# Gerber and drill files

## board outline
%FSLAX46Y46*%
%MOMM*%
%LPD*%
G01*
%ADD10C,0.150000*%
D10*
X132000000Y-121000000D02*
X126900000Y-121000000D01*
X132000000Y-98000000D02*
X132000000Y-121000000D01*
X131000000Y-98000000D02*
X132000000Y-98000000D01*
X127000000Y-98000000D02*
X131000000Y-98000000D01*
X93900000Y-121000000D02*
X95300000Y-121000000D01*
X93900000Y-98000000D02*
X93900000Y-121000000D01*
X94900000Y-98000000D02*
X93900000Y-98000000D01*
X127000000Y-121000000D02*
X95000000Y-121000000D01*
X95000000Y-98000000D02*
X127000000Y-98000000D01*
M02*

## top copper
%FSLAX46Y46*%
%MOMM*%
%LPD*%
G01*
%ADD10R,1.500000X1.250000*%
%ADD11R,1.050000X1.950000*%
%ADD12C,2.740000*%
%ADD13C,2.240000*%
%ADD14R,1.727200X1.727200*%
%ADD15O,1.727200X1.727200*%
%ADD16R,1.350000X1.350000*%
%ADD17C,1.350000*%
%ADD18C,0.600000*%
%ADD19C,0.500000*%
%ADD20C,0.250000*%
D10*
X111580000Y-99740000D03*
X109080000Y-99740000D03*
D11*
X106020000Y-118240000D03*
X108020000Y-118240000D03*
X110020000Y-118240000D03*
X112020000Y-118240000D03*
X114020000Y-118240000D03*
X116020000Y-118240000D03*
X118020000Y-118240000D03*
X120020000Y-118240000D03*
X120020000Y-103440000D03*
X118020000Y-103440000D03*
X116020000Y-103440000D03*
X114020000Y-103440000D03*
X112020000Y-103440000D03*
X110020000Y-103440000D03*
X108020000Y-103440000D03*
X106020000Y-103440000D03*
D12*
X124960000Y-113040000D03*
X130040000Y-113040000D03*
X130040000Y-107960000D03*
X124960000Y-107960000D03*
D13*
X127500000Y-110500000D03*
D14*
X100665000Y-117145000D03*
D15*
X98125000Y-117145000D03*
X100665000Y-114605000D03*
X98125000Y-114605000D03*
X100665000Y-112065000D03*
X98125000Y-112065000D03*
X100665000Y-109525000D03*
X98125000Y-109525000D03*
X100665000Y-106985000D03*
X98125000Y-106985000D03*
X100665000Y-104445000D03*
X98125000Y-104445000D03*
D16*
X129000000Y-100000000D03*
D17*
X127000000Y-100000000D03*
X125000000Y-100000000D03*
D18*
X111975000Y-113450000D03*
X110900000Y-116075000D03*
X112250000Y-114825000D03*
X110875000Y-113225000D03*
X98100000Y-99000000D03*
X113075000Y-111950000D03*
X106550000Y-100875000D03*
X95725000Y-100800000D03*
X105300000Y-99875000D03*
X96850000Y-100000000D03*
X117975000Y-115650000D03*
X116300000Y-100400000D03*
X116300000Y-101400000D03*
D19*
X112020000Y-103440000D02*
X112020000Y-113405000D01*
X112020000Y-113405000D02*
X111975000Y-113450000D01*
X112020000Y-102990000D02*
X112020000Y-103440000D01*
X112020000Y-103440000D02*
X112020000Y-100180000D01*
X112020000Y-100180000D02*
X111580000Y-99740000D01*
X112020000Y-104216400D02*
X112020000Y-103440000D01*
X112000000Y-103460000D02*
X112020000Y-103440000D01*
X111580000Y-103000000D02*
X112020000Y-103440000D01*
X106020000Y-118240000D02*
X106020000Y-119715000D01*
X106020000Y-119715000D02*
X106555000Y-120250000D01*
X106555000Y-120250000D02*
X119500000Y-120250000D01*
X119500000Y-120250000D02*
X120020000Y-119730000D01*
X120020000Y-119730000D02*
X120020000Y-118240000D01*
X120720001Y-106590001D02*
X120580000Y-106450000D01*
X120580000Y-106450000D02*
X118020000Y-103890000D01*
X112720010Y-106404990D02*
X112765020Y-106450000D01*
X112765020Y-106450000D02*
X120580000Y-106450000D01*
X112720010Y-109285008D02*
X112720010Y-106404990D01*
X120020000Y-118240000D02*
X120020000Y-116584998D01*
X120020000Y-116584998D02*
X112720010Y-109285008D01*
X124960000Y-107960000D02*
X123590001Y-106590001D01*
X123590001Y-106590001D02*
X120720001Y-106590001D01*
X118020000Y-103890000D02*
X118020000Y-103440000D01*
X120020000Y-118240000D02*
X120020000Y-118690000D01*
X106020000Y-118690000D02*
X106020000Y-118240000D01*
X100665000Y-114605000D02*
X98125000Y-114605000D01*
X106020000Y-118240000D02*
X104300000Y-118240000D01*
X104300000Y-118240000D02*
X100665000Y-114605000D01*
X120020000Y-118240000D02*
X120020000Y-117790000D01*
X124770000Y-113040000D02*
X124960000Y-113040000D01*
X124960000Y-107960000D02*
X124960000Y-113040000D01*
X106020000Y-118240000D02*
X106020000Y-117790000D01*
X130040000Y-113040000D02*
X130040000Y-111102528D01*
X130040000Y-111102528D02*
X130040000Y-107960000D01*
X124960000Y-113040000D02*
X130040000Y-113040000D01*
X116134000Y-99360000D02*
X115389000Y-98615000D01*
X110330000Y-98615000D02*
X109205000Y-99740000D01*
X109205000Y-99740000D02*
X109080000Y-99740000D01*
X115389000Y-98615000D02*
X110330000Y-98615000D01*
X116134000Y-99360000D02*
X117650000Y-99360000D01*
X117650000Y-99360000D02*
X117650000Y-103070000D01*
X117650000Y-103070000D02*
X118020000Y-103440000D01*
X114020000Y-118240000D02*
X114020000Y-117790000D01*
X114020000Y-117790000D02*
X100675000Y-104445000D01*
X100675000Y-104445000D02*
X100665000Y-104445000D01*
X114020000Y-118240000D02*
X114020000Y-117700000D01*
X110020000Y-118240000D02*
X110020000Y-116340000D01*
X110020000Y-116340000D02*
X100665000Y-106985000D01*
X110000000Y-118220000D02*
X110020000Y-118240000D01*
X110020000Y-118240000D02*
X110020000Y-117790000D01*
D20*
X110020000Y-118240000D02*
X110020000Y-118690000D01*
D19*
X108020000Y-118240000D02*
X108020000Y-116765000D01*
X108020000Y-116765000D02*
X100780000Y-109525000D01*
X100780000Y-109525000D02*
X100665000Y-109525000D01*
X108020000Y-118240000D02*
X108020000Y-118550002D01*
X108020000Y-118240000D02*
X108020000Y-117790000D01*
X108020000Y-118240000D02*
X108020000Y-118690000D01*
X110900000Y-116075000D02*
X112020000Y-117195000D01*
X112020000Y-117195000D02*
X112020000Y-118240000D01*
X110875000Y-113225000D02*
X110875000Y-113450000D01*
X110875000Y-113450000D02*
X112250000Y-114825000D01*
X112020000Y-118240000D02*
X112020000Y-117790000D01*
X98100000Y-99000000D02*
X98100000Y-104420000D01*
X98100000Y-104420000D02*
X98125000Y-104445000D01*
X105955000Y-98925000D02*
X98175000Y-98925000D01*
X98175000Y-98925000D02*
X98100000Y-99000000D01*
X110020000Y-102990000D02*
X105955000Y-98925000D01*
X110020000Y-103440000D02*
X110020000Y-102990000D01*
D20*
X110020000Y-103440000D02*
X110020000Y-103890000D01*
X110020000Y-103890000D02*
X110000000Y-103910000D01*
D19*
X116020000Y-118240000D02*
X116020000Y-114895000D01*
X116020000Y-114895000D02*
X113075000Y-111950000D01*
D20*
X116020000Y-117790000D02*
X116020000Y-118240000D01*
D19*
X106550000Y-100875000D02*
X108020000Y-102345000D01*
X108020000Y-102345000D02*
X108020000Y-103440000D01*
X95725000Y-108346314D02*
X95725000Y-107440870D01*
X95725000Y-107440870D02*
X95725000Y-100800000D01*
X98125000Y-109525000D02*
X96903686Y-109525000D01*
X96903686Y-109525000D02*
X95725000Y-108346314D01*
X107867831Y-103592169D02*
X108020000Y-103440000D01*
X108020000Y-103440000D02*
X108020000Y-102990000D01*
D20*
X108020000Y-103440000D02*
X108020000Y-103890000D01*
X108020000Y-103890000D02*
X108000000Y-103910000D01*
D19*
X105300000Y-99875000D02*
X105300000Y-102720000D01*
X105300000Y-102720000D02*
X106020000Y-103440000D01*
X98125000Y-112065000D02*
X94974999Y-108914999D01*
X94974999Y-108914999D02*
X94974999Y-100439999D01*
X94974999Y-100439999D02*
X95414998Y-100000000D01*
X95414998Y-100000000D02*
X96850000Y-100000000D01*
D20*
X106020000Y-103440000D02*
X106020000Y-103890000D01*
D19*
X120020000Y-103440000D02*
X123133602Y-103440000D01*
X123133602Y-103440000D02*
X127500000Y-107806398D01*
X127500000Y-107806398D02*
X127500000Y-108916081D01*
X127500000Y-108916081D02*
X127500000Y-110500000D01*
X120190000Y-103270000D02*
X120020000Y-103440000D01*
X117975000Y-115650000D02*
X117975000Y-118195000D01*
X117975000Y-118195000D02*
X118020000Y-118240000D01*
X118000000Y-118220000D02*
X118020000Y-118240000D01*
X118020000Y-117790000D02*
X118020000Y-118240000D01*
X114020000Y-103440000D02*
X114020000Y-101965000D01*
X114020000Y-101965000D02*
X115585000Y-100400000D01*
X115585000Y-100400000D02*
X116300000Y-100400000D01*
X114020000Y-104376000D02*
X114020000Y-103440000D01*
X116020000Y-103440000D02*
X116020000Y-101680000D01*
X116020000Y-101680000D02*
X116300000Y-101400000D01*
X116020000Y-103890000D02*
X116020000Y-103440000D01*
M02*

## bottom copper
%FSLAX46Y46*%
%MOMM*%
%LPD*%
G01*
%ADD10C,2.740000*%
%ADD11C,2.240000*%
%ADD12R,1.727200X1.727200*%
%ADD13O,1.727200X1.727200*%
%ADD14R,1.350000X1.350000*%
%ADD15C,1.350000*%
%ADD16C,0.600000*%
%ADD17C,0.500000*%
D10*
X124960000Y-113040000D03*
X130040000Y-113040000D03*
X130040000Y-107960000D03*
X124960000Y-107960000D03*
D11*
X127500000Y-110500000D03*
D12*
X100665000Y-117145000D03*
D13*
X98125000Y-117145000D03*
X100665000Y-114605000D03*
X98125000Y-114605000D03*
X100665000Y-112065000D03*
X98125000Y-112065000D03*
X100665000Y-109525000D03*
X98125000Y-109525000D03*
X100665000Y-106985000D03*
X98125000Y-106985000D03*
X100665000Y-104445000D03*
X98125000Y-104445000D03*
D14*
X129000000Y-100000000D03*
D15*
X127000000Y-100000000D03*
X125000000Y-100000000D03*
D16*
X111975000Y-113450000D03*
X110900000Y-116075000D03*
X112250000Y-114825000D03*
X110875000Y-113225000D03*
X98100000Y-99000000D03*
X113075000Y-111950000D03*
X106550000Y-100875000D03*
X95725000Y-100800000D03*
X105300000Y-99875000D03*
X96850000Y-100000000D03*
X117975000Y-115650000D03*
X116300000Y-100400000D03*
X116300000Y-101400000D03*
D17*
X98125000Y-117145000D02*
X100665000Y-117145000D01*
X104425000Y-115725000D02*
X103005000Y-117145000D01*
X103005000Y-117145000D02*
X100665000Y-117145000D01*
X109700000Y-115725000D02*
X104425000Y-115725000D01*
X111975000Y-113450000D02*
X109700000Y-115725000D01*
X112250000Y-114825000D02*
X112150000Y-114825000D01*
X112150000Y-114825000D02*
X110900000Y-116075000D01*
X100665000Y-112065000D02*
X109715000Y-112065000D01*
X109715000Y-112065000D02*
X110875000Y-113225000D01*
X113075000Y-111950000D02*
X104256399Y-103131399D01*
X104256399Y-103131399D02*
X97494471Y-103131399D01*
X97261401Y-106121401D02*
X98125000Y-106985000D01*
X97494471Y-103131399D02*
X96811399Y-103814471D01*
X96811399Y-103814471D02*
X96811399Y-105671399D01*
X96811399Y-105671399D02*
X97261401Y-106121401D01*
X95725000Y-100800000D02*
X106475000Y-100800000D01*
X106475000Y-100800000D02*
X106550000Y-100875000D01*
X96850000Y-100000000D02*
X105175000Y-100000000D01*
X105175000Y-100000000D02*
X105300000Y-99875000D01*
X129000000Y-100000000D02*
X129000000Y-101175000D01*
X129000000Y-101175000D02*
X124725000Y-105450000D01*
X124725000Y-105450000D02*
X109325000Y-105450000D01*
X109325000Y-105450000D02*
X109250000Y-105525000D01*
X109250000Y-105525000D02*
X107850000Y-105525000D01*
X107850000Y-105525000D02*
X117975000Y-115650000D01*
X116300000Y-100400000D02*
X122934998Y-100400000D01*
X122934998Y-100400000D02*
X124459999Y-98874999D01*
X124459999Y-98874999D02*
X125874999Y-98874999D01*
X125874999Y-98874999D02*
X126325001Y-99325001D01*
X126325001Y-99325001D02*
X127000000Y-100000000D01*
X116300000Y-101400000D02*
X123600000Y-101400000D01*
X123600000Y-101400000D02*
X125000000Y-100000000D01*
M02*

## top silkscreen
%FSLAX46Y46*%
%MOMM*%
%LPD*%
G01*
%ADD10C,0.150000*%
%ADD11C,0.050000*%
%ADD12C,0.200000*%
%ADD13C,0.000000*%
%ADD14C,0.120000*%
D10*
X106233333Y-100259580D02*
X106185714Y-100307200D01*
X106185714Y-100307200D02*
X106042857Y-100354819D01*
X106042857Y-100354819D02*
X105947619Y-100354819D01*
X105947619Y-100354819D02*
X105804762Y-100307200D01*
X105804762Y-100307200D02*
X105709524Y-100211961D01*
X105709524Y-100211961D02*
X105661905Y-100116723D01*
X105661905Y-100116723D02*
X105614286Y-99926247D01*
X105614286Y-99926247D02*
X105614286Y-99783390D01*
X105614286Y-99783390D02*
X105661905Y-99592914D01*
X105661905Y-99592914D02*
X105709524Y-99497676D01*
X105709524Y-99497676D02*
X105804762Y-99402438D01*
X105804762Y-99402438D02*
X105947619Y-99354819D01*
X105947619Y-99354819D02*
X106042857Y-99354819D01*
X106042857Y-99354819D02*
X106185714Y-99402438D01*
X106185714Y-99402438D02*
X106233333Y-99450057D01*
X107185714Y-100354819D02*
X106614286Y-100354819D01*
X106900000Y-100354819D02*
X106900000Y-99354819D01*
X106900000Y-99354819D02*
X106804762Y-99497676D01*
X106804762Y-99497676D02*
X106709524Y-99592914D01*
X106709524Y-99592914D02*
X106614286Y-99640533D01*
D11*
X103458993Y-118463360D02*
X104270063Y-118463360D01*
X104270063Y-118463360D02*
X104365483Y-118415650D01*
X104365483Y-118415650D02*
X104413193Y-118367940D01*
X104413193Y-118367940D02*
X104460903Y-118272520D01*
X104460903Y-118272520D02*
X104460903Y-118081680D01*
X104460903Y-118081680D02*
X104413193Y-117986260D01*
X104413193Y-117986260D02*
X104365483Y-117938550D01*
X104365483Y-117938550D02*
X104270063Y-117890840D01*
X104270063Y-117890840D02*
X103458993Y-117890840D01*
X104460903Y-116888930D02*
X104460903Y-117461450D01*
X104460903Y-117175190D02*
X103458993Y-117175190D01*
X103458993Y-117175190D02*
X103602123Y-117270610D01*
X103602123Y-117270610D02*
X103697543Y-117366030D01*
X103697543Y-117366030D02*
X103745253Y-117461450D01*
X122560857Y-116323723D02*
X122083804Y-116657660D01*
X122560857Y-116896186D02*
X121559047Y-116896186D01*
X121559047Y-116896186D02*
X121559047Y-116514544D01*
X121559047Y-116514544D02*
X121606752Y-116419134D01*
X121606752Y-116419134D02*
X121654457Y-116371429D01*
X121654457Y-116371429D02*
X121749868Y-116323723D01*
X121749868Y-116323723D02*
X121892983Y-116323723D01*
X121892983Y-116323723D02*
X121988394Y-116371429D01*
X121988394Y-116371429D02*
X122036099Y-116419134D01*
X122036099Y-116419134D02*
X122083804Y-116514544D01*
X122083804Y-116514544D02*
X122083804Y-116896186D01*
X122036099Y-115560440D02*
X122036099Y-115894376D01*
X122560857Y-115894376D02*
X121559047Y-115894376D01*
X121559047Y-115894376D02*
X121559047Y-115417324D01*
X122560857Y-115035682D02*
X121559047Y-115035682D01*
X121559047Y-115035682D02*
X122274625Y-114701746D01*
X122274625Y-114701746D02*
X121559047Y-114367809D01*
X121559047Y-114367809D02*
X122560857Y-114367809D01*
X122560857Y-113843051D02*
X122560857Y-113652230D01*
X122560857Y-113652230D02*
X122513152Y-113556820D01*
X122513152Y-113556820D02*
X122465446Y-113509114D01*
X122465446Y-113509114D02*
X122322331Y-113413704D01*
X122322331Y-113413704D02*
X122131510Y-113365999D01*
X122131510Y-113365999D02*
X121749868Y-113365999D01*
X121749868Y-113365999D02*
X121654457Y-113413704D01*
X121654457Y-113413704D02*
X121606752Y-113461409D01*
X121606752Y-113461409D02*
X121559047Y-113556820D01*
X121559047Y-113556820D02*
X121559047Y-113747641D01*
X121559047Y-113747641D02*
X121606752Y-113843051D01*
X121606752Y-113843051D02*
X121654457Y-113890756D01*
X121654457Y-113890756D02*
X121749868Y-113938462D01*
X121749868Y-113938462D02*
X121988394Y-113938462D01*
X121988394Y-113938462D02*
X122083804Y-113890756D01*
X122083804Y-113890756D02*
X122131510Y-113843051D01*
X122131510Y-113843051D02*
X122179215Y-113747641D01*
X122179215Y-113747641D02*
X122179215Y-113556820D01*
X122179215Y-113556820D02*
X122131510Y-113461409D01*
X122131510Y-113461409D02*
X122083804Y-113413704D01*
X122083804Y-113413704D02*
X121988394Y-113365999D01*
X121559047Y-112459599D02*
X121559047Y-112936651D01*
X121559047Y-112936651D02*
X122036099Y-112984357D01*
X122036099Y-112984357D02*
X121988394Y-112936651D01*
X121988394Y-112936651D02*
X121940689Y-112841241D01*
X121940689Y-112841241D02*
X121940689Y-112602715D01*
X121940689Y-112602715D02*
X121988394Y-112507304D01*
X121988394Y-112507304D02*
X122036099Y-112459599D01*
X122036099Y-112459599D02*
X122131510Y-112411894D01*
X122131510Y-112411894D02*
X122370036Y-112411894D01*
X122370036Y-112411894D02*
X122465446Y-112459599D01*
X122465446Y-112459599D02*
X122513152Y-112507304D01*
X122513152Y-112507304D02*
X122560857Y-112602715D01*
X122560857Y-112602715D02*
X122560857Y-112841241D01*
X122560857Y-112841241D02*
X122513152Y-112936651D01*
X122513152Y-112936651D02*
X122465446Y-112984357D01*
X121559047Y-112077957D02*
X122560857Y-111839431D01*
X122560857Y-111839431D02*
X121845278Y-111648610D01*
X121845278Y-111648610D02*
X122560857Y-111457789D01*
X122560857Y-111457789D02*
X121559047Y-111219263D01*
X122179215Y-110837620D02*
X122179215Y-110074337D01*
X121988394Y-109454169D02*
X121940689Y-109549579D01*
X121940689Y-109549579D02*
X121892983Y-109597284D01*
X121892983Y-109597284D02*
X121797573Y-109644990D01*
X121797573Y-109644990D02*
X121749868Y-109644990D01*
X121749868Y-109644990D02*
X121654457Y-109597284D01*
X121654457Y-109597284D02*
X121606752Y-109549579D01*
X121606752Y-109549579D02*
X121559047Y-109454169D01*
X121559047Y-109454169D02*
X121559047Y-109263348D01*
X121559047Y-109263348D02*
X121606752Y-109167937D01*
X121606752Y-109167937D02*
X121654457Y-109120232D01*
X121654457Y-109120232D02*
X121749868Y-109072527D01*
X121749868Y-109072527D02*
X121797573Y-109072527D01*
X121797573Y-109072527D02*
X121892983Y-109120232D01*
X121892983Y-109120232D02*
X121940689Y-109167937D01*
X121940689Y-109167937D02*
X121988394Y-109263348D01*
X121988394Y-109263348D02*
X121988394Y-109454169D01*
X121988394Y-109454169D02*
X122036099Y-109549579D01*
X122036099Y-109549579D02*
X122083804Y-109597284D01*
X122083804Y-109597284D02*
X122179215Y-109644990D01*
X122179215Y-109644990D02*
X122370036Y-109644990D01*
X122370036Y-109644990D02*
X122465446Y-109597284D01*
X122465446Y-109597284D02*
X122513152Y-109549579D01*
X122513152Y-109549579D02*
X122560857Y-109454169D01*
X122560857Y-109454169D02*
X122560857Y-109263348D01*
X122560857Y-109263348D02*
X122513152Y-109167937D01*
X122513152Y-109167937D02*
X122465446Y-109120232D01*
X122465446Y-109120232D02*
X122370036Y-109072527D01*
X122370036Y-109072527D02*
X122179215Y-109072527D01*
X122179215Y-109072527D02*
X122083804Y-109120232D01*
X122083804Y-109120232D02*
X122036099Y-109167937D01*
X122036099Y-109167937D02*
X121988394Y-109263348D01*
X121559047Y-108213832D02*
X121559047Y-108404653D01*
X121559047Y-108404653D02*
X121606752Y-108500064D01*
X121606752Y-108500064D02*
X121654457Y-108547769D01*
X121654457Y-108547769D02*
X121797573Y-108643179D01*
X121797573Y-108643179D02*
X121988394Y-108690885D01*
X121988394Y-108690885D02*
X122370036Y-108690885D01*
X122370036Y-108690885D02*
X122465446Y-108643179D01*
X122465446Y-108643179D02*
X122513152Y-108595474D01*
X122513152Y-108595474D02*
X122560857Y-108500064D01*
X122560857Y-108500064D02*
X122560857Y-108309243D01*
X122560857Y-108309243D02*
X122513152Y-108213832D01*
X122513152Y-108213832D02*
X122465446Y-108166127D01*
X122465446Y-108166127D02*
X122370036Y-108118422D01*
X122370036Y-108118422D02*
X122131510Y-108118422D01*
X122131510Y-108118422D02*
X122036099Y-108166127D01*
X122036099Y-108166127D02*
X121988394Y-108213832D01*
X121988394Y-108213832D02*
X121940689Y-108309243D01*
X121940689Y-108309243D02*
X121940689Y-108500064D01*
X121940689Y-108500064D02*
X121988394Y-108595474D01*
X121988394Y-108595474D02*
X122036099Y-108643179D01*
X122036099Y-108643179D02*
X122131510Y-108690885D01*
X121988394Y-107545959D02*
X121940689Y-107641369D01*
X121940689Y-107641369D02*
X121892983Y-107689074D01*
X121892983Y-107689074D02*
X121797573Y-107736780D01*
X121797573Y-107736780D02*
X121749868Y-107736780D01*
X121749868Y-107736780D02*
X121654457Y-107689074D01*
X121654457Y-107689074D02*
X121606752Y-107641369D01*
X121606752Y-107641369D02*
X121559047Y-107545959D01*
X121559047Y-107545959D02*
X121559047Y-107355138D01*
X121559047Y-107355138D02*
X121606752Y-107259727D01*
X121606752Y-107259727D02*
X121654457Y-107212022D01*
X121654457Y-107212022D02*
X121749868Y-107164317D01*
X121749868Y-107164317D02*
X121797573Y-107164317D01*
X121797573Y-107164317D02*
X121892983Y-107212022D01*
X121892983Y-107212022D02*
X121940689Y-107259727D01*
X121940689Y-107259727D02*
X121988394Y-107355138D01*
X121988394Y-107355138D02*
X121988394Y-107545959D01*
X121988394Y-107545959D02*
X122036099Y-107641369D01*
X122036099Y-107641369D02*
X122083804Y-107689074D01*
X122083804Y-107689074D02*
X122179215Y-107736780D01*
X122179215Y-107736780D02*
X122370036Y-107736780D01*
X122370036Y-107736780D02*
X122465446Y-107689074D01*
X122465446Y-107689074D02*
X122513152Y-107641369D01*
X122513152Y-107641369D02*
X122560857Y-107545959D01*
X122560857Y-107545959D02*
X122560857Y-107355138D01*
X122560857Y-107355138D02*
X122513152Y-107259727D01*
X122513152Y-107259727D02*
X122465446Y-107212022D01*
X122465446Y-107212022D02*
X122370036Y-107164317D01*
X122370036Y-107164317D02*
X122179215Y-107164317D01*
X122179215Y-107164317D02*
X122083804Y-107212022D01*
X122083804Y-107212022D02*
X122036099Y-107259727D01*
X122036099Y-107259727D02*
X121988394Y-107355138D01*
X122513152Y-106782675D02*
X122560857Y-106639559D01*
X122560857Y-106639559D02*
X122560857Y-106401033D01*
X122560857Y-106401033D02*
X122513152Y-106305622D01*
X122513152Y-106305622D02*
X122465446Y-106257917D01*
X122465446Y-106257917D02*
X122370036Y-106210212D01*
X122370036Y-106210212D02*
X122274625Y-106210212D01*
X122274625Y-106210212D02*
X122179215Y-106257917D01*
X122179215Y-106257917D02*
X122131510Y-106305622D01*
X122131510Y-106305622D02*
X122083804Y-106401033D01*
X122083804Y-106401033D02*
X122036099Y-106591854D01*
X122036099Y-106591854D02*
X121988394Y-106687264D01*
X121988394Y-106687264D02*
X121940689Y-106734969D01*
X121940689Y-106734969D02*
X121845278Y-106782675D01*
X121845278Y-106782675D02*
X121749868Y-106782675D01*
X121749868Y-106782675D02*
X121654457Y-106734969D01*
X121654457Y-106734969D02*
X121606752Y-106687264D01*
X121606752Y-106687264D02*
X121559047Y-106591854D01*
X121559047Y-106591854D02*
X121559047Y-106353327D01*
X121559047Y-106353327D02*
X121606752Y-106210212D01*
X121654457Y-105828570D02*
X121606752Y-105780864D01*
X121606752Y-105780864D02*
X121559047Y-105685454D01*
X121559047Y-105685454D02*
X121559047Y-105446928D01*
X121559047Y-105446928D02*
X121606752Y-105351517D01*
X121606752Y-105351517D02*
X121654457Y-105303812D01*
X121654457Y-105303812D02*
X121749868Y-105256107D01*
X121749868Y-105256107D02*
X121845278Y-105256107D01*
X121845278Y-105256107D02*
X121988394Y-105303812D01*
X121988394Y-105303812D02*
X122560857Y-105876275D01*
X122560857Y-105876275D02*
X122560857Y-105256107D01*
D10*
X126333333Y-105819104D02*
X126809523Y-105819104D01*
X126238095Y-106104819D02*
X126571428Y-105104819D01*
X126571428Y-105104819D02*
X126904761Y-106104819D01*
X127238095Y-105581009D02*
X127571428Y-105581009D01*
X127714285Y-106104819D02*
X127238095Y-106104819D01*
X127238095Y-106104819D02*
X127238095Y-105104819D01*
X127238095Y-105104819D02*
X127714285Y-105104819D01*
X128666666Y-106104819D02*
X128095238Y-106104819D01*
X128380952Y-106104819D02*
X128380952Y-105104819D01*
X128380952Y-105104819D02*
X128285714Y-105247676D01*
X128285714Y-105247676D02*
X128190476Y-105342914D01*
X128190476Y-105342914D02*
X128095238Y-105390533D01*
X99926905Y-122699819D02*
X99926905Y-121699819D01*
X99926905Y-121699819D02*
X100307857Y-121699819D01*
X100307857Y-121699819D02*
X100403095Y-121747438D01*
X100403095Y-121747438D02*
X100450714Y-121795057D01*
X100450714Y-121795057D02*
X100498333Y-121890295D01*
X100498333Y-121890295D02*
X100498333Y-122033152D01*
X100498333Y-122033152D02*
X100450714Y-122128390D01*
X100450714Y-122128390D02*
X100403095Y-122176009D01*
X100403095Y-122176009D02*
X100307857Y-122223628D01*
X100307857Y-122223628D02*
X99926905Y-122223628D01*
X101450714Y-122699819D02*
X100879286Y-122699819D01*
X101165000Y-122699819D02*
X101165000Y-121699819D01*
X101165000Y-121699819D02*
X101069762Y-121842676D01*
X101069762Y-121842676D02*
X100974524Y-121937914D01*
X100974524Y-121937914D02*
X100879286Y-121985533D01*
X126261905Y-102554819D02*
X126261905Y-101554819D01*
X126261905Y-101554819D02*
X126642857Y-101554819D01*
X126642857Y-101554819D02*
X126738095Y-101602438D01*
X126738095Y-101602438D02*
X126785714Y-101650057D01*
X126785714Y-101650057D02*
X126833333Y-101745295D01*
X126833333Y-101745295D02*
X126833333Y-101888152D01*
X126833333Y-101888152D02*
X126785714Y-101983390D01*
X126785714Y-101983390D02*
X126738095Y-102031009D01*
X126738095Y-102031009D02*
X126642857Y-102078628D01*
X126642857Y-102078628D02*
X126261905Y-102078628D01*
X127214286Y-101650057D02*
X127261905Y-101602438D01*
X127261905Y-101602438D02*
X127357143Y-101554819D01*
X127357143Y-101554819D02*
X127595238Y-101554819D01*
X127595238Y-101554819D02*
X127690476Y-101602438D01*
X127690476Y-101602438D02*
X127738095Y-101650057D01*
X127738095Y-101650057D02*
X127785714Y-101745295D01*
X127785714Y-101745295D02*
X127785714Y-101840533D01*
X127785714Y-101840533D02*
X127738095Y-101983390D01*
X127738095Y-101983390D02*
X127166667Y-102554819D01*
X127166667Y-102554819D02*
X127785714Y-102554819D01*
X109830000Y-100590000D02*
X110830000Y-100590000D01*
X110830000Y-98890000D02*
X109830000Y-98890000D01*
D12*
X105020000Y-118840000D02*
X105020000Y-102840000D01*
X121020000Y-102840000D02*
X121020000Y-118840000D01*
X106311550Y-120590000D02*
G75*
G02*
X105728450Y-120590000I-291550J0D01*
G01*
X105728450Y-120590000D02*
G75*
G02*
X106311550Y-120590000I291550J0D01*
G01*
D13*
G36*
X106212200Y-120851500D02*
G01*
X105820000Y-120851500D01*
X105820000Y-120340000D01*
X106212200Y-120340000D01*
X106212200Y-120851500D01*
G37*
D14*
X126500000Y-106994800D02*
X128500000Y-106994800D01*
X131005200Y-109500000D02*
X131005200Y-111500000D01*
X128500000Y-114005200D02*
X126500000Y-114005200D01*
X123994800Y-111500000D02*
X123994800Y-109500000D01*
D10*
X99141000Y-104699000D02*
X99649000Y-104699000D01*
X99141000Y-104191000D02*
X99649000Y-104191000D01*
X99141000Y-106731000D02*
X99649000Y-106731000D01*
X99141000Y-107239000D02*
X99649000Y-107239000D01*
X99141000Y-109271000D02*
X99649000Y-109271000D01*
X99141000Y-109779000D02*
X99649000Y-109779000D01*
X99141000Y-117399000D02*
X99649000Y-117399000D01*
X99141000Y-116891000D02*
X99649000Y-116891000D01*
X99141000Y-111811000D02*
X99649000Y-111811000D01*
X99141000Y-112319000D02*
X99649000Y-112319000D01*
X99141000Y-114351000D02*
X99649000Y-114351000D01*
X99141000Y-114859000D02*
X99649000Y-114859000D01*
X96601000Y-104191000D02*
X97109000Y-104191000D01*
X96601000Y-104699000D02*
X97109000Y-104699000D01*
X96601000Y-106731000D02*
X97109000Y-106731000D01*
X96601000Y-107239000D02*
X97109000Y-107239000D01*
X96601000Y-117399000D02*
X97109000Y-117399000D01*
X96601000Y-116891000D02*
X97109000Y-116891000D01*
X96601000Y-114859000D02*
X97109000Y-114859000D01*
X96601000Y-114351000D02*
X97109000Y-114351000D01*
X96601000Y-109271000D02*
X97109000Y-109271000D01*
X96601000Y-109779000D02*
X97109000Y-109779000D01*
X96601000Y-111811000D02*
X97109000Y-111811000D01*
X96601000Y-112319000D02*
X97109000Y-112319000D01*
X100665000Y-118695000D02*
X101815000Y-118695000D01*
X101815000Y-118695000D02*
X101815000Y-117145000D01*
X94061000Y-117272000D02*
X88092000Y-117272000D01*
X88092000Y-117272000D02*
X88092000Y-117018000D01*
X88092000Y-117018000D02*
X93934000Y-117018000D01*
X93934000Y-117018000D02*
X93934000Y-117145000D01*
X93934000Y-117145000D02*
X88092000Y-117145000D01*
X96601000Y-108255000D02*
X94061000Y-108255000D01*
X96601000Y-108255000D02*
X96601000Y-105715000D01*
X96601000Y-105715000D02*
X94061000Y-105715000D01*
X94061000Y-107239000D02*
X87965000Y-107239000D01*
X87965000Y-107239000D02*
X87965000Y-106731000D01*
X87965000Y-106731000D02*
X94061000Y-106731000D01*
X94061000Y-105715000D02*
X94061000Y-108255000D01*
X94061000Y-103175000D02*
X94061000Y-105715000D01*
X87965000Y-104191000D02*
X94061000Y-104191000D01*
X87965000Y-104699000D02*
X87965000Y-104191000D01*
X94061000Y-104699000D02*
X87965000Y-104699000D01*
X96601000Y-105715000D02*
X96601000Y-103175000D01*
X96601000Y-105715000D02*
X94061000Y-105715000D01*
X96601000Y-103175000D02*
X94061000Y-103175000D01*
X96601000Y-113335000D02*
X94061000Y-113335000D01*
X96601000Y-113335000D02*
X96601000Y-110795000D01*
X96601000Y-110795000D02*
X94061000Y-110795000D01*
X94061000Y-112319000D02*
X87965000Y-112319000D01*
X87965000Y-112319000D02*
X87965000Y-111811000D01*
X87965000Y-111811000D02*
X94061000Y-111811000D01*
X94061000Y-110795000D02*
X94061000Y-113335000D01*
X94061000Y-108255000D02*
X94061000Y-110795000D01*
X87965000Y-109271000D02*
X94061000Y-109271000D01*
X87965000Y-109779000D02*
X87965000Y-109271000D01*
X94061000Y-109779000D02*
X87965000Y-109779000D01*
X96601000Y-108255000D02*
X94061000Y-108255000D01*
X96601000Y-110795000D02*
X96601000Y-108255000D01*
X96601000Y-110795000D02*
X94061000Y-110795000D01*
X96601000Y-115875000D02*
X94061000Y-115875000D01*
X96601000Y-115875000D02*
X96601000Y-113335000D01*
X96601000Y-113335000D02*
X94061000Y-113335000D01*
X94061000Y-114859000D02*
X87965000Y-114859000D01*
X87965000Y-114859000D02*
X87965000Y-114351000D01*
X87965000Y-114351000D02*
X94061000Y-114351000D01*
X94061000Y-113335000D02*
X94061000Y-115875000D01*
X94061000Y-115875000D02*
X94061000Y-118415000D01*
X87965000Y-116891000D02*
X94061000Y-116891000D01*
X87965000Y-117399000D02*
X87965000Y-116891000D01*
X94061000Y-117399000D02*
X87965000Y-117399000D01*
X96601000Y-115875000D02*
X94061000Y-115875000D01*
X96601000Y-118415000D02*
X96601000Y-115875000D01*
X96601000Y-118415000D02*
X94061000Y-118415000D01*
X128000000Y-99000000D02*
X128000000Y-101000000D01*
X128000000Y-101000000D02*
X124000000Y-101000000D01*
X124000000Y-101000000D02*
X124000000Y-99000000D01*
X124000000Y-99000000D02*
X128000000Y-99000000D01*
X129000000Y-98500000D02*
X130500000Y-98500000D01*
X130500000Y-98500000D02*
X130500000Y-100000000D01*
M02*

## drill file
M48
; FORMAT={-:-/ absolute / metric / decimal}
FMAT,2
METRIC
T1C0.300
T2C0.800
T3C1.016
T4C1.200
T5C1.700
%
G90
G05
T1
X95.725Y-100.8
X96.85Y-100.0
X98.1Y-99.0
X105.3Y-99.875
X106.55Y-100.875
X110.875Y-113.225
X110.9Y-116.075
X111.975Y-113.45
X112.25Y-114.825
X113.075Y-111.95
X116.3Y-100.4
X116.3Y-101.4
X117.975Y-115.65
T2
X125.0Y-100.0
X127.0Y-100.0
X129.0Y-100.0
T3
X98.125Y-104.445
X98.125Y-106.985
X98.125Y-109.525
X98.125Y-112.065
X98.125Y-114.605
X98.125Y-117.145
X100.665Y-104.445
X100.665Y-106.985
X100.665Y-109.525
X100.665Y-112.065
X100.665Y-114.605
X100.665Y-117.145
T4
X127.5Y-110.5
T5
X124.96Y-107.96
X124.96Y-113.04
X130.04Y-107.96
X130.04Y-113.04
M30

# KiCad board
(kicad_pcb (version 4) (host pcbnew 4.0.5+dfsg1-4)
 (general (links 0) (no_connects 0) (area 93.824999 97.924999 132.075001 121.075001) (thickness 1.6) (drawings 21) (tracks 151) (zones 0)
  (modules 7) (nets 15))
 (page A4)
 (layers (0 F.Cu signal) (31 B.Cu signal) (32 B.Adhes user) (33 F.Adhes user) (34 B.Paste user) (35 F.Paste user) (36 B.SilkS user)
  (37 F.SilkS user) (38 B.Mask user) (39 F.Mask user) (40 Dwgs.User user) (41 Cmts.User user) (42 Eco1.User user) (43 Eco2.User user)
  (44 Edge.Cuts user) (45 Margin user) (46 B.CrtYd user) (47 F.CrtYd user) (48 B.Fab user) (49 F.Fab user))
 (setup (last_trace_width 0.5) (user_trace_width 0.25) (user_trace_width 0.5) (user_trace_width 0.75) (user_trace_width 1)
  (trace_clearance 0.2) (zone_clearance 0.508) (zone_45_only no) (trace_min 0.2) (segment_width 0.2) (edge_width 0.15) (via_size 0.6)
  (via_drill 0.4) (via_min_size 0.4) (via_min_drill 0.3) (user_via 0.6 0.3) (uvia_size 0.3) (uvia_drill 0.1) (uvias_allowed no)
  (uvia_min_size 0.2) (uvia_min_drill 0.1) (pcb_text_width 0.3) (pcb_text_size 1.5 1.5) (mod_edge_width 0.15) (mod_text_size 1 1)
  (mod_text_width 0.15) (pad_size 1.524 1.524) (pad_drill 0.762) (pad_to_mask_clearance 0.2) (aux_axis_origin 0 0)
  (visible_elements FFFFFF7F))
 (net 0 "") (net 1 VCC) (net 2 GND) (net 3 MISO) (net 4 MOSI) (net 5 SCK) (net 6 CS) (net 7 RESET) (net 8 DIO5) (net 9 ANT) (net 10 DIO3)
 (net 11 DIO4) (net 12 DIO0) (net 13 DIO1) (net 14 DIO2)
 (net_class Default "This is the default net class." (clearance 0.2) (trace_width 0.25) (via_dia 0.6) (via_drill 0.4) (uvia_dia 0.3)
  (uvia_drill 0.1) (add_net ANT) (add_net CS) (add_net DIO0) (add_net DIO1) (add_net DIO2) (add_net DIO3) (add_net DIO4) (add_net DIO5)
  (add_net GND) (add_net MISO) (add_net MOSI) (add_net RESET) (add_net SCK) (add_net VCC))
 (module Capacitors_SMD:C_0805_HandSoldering (layer F.Cu) (at 110.33 99.74 180)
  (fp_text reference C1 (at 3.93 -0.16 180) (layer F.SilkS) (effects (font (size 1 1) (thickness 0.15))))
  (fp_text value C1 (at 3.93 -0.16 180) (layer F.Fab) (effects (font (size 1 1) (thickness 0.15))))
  (fp_line (start 0.5 -0.85) (end -0.5 -0.85) (layer F.SilkS) (width 0.15))
  (fp_line (start -0.5 0.85) (end 0.5 0.85) (layer F.SilkS) (width 0.15))
  (pad 1 smd rect (at -1.25 0 180) (size 1.5 1.25) (layers F.Cu F.Paste F.Mask) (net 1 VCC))
  (pad 2 smd rect (at 1.25 0 180) (size 1.5 1.25) (layers F.Cu F.Paste F.Mask) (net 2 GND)))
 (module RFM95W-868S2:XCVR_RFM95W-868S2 (layer F.Cu) (at 113.02 110.84 90)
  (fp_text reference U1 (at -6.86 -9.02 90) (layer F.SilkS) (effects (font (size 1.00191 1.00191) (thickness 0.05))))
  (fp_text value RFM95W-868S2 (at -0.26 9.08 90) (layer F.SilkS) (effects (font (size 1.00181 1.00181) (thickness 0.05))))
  (fp_line (start -8 -8) (end 8 -8) (layer F.SilkS) (width 0.2)) (fp_line (start 8 8) (end -8 8) (layer F.SilkS) (width 0.2))
  (fp_circle (center -9.75 -7) (end -9.45845 -7) (layer F.SilkS) (width 0.2))
  (fp_poly (pts (xy -10.0115 -7.2) (xy -9.5 -7.2) (xy -9.5 -6.8078) (xy -10.0115 -6.8078)) (layer F.SilkS) (width 0))
  (pad 1 smd rect (at -7.4 -7 90) (size 1.95 1.05) (layers F.Cu F.Paste F.Mask) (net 2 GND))
  (pad 2 smd rect (at -7.4 -5 90) (size 1.95 1.05) (layers F.Cu F.Paste F.Mask) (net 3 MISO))
  (pad 3 smd rect (at -7.4 -3 90) (size 1.95 1.05) (layers F.Cu F.Paste F.Mask) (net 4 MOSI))
  (pad 4 smd rect (at -7.4 -1 90) (size 1.95 1.05) (layers F.Cu F.Paste F.Mask) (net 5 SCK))
  (pad 5 smd rect (at -7.4 1 90) (size 1.95 1.05) (layers F.Cu F.Paste F.Mask) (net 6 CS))
  (pad 6 smd rect (at -7.4 3 90) (size 1.95 1.05) (layers F.Cu F.Paste F.Mask) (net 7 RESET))
  (pad 7 smd rect (at -7.4 5 90) (size 1.95 1.05) (layers F.Cu F.Paste F.Mask) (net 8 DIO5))
  (pad 8 smd rect (at -7.4 7 90) (size 1.95 1.05) (layers F.Cu F.Paste F.Mask) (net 2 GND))
  (pad 9 smd rect (at 7.4 7 270) (size 1.95 1.05) (layers F.Cu F.Paste F.Mask) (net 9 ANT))
  (pad 10 smd rect (at 7.4 5 270) (size 1.95 1.05) (layers F.Cu F.Paste F.Mask) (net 2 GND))
  (pad 11 smd rect (at 7.4 3 270) (size 1.95 1.05) (layers F.Cu F.Paste F.Mask) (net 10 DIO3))
  (pad 12 smd rect (at 7.4 1 270) (size 1.95 1.05) (layers F.Cu F.Paste F.Mask) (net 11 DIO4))
  (pad 13 smd rect (at 7.4 -1 270) (size 1.95 1.05) (layers F.Cu F.Paste F.Mask) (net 1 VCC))
  (pad 14 smd rect (at 7.4 -3 270) (size 1.95 1.05) (layers F.Cu F.Paste F.Mask) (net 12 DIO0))
  (pad 15 smd rect (at 7.4 -5 270) (size 1.95 1.05) (layers F.Cu F.Paste F.Mask) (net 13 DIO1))
  (pad 16 smd rect (at 7.4 -7 270) (size 1.95 1.05) (layers F.Cu F.Paste F.Mask) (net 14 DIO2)))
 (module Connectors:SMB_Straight (layer F.Cu) (at 127.5 110.5)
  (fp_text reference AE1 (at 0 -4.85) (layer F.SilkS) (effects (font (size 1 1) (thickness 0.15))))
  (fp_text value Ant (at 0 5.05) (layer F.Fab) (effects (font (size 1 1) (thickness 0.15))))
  (fp_line (start -1 -3.5052) (end 1 -3.5052) (layer F.SilkS) (width 0.12))
  (fp_line (start 3.5052 -1) (end 3.5052 1) (layer F.SilkS) (width 0.12))
  (fp_line (start 1 3.5052) (end -1 3.5052) (layer F.SilkS) (width 0.12))
  (fp_line (start -3.5052 1) (end -3.5052 -1) (layer F.SilkS) (width 0.12))
  (pad 2 thru_hole circle (at -2.54 2.54) (size 2.74 2.74) (drill 1.7) (layers *.Cu *.Mask) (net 2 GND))
  (pad 2 thru_hole circle (at 2.54 2.54) (size 2.74 2.74) (drill 1.7) (layers *.Cu *.Mask) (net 2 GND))
  (pad 2 thru_hole circle (at 2.54 -2.54) (size 2.74 2.74) (drill 1.7) (layers *.Cu *.Mask) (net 2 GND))
  (pad 2 thru_hole circle (at -2.54 -2.54) (size 2.74 2.74) (drill 1.7) (layers *.Cu *.Mask) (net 2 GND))
  (pad 1 thru_hole circle (at 0 0) (size 2.24 2.24) (drill 1.2) (layers *.Cu *.Mask) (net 9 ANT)))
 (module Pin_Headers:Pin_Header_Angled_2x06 (layer F.Cu) (at 100.665 117.145 180)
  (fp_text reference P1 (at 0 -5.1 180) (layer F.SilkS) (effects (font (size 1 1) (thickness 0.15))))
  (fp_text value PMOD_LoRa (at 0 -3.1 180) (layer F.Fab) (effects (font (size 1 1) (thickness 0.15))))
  (fp_line (start 1.524 12.446) (end 1.016 12.446) (layer F.SilkS) (width 0.15))
  (fp_line (start 1.524 12.954) (end 1.016 12.954) (layer F.SilkS) (width 0.15))
  (fp_line (start 1.524 10.414) (end 1.016 10.414) (layer F.SilkS) (width 0.15))
  (fp_line (start 1.524 9.906) (end 1.016 9.906) (layer F.SilkS) (width 0.15))
  (fp_line (start 1.524 7.874) (end 1.016 7.874) (layer F.SilkS) (width 0.15))
  (fp_line (start 1.524 7.366) (end 1.016 7.366) (layer F.SilkS) (width 0.15))
  (fp_line (start 1.524 -0.254) (end 1.016 -0.254) (layer F.SilkS) (width 0.15))
  (fp_line (start 1.524 0.254) (end 1.016 0.254) (layer F.SilkS) (width 0.15))
  (fp_line (start 1.524 5.334) (end 1.016 5.334) (layer F.SilkS) (width 0.15))
  (fp_line (start 1.524 4.826) (end 1.016 4.826) (layer F.SilkS) (width 0.15))
  (fp_line (start 1.524 2.794) (end 1.016 2.794) (layer F.SilkS) (width 0.15))
  (fp_line (start 1.524 2.286) (end 1.016 2.286) (layer F.SilkS) (width 0.15))
  (fp_line (start 4.064 12.954) (end 3.556 12.954) (layer F.SilkS) (width 0.15))
  (fp_line (start 4.064 12.446) (end 3.556 12.446) (layer F.SilkS) (width 0.15))
  (fp_line (start 4.064 10.414) (end 3.556 10.414) (layer F.SilkS) (width 0.15))
  (fp_line (start 4.064 9.906) (end 3.556 9.906) (layer F.SilkS) (width 0.15))
  (fp_line (start 4.064 -0.254) (end 3.556 -0.254) (layer F.SilkS) (width 0.15))
  (fp_line (start 4.064 0.254) (end 3.556 0.254) (layer F.SilkS) (width 0.15))
  (fp_line (start 4.064 2.286) (end 3.556 2.286) (layer F.SilkS) (width 0.15))
  (fp_line (start 4.064 2.794) (end 3.556 2.794) (layer F.SilkS) (width 0.15))
  (fp_line (start 4.064 7.874) (end 3.556 7.874) (layer F.SilkS) (width 0.15))
  (fp_line (start 4.064 7.366) (end 3.556 7.366) (layer F.SilkS) (width 0.15))
  (fp_line (start 4.064 5.334) (end 3.556 5.334) (layer F.SilkS) (width 0.15))
  (fp_line (start 4.064 4.826) (end 3.556 4.826) (layer F.SilkS) (width 0.15))
  (fp_line (start 0 -1.55) (end -1.15 -1.55) (layer F.SilkS) (width 0.15))
  (fp_line (start -1.15 -1.55) (end -1.15 0) (layer F.SilkS) (width 0.15))
  (fp_line (start 6.604 -0.127) (end 12.573 -0.127) (layer F.SilkS) (width 0.15))
  (fp_line (start 12.573 -0.127) (end 12.573 0.127) (layer F.SilkS) (width 0.15))
  (fp_line (start 12.573 0.127) (end 6.731 0.127) (layer F.SilkS) (width 0.15))
  (fp_line (start 6.731 0.127) (end 6.731 0) (layer F.SilkS) (width 0.15))
  (fp_line (start 6.731 0) (end 12.573 0) (layer F.SilkS) (width 0.15))
  (fp_line (start 4.064 8.89) (end 6.604 8.89) (layer F.SilkS) (width 0.15))
  (fp_line (start 4.064 8.89) (end 4.064 11.43) (layer F.SilkS) (width 0.15))
  (fp_line (start 4.064 11.43) (end 6.604 11.43) (layer F.SilkS) (width 0.15))
  (fp_line (start 6.604 9.906) (end 12.7 9.906) (layer F.SilkS) (width 0.15))
  (fp_line (start 12.7 9.906) (end 12.7 10.414) (layer F.SilkS) (width 0.15))
  (fp_line (start 12.7 10.414) (end 6.604 10.414) (layer F.SilkS) (width 0.15))
  (fp_line (start 6.604 11.43) (end 6.604 8.89) (layer F.SilkS) (width 0.15))
  (fp_line (start 6.604 13.97) (end 6.604 11.43) (layer F.SilkS) (width 0.15))
  (fp_line (start 12.7 12.954) (end 6.604 12.954) (layer F.SilkS) (width 0.15))
  (fp_line (start 12.7 12.446) (end 12.7 12.954) (layer F.SilkS) (width 0.15))
  (fp_line (start 6.604 12.446) (end 12.7 12.446) (layer F.SilkS) (width 0.15))
  (fp_line (start 4.064 11.43) (end 4.064 13.97) (layer F.SilkS) (width 0.15))
  (fp_line (start 4.064 11.43) (end 6.604 11.43) (layer F.SilkS) (width 0.15))
  (fp_line (start 4.064 13.97) (end 6.604 13.97) (layer F.SilkS) (width 0.15))
  (fp_line (start 4.064 3.81) (end 6.604 3.81) (layer F.SilkS) (width 0.15))
  (fp_line (start 4.064 3.81) (end 4.064 6.35) (layer F.SilkS) (width 0.15))
  (fp_line (start 4.064 6.35) (end 6.604 6.35) (layer F.SilkS) (width 0.15))
  (fp_line (start 6.604 4.826) (end 12.7 4.826) (layer F.SilkS) (width 0.15))
  (fp_line (start 12.7 4.826) (end 12.7 5.334) (layer F.SilkS) (width 0.15))
  (fp_line (start 12.7 5.334) (end 6.604 5.334) (layer F.SilkS) (width 0.15))
  (fp_line (start 6.604 6.35) (end 6.604 3.81) (layer F.SilkS) (width 0.15))
  (fp_line (start 6.604 8.89) (end 6.604 6.35) (layer F.SilkS) (width 0.15))
  (fp_line (start 12.7 7.874) (end 6.604 7.874) (layer F.SilkS) (width 0.15))
  (fp_line (start 12.7 7.366) (end 12.7 7.874) (layer F.SilkS) (width 0.15))
  (fp_line (start 6.604 7.366) (end 12.7 7.366) (layer F.SilkS) (width 0.15))
  (fp_line (start 4.064 8.89) (end 6.604 8.89) (layer F.SilkS) (width 0.15))
  (fp_line (start 4.064 6.35) (end 4.064 8.89) (layer F.SilkS) (width 0.15))
  (fp_line (start 4.064 6.35) (end 6.604 6.35) (layer F.SilkS) (width 0.15))
  (fp_line (start 4.064 1.27) (end 6.604 1.27) (layer F.SilkS) (width 0.15))
  (fp_line (start 4.064 1.27) (end 4.064 3.81) (layer F.SilkS) (width 0.15))
  (fp_line (start 4.064 3.81) (end 6.604 3.81) (layer F.SilkS) (width 0.15))
  (fp_line (start 6.604 2.286) (end 12.7 2.286) (layer F.SilkS) (width 0.15))
  (fp_line (start 12.7 2.286) (end 12.7 2.794) (layer F.SilkS) (width 0.15))
  (fp_line (start 12.7 2.794) (end 6.604 2.794) (layer F.SilkS) (width 0.15))
  (fp_line (start 6.604 3.81) (end 6.604 1.27) (layer F.SilkS) (width 0.15))
  (fp_line (start 6.604 1.27) (end 6.604 -1.27) (layer F.SilkS) (width 0.15))
  (fp_line (start 12.7 0.254) (end 6.604 0.254) (layer F.SilkS) (width 0.15))
  (fp_line (start 12.7 -0.254) (end 12.7 0.254) (layer F.SilkS) (width 0.15))
  (fp_line (start 6.604 -0.254) (end 12.7 -0.254) (layer F.SilkS) (width 0.15))
  (fp_line (start 4.064 1.27) (end 6.604 1.27) (layer F.SilkS) (width 0.15))
  (fp_line (start 4.064 -1.27) (end 4.064 1.27) (layer F.SilkS) (width 0.15))
  (fp_line (start 4.064 -1.27) (end 6.604 -1.27) (layer F.SilkS) (width 0.15))
  (pad 1 thru_hole rect (at 0 0 180) (size 1.7272 1.7272) (drill 1.016) (layers *.Cu *.Mask) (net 1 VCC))
  (pad 2 thru_hole oval (at 2.54 0 180) (size 1.7272 1.7272) (drill 1.016) (layers *.Cu *.Mask) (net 1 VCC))
  (pad 3 thru_hole oval (at 0 2.54 180) (size 1.7272 1.7272) (drill 1.016) (layers *.Cu *.Mask) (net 2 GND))
  (pad 4 thru_hole oval (at 2.54 2.54 180) (size 1.7272 1.7272) (drill 1.016) (layers *.Cu *.Mask) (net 2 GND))
  (pad 5 thru_hole oval (at 0 5.08 180) (size 1.7272 1.7272) (drill 1.016) (layers *.Cu *.Mask) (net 5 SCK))
  (pad 6 thru_hole oval (at 2.54 5.08 180) (size 1.7272 1.7272) (drill 1.016) (layers *.Cu *.Mask) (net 14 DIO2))
  (pad 7 thru_hole oval (at 0 7.62 180) (size 1.7272 1.7272) (drill 1.016) (layers *.Cu *.Mask) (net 3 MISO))
  (pad 8 thru_hole oval (at 2.54 7.62 180) (size 1.7272 1.7272) (drill 1.016) (layers *.Cu *.Mask) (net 13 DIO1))
  (pad 9 thru_hole oval (at 0 10.16 180) (size 1.7272 1.7272) (drill 1.016) (layers *.Cu *.Mask) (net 4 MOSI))
  (pad 10 thru_hole oval (at 2.54 10.16 180) (size 1.7272 1.7272) (drill 1.016) (layers *.Cu *.Mask) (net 7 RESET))
  (pad 11 thru_hole oval (at 0 12.7 180) (size 1.7272 1.7272) (drill 1.016) (layers *.Cu *.Mask) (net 6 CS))
  (pad 12 thru_hole oval (at 2.54 12.7 180) (size 1.7272 1.7272) (drill 1.016) (layers *.Cu *.Mask) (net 12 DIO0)))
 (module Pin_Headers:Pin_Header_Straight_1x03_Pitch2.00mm (layer F.Cu) (at 129 100 270)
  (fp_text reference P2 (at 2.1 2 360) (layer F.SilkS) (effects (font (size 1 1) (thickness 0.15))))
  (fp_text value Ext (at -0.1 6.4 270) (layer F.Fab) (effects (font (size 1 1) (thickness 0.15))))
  (fp_line (start -1 1) (end 1 1) (layer F.SilkS) (width 0.15)) (fp_line (start 1 1) (end 1 5) (layer F.SilkS) (width 0.15))
  (fp_line (start 1 5) (end -1 5) (layer F.SilkS) (width 0.15))
  (fp_line (start -1 5) (end -1 1) (layer F.SilkS) (width 0.15))
  (fp_line (start -1.5 0) (end -1.5 -1.5) (layer F.SilkS) (width 0.15))
  (fp_line (start -1.5 -1.5) (end 0 -1.5) (layer F.SilkS) (width 0.15))
  (pad 1 thru_hole rect (at 0 0 270) (size 1.35 1.35) (drill 0.8) (layers *.Cu *.Mask) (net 8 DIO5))
  (pad 2 thru_hole circle (at 0 2 270) (size 1.35 1.35) (drill 0.8) (layers *.Cu *.Mask) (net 11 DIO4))
  (pad 3 thru_hole circle (at 0 4 270) (size 1.35 1.35) (drill 0.8) (layers *.Cu *.Mask) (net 10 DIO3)))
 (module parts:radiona (layer B.Cu) (at 113.4 101.25 180)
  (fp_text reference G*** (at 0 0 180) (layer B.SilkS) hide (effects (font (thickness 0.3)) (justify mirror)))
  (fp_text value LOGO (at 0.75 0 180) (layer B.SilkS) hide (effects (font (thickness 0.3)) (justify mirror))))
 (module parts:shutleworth (layer B.Cu) (at 118.55 117.475 180)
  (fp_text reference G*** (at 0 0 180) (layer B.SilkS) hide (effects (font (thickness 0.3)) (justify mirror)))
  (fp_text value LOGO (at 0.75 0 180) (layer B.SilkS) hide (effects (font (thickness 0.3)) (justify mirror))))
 (gr_line (start 132 121) (end 126.9 121) (layer Edge.Cuts) (width 0.15))
 (gr_line (start 132 98) (end 132 121) (layer Edge.Cuts) (width 0.15))
 (gr_line (start 131 98) (end 132 98) (layer Edge.Cuts) (width 0.15))
 (gr_line (start 127 98) (end 131 98) (layer Edge.Cuts) (width 0.15))
 (gr_line (start 93.9 121) (end 95.3 121) (layer Edge.Cuts) (width 0.15))
 (gr_line (start 93.9 98) (end 93.9 121) (layer Edge.Cuts) (width 0.15))
 (gr_line (start 94.9 98) (end 93.9 98) (layer Edge.Cuts) (width 0.15))
 (gr_line (start 127 121) (end 95 121) (layer Edge.Cuts) (width 0.15))
 (gr_line (start 95 98) (end 127 98) (layer Edge.Cuts) (width 0.15))
 (segment (start 98.125 117.145) (end 100.665 117.145) (width 0.5) (layer B.Cu) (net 1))
 (segment (start 104.425 115.725) (end 103.005 117.145) (width 0.5) (layer B.Cu) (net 1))
 (segment (start 103.005 117.145) (end 100.665 117.145) (width 0.5) (layer B.Cu) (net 1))
 (segment (start 109.7 115.725) (end 104.425 115.725) (width 0.5) (layer B.Cu) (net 1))
 (segment (start 111.975 113.45) (end 109.7 115.725) (width 0.5) (layer B.Cu) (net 1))
 (segment (start 112.02 103.44) (end 112.02 113.405) (width 0.5) (layer F.Cu) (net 1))
 (segment (start 112.02 113.405) (end 111.975 113.45) (width 0.5) (layer F.Cu) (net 1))
 (via (at 111.975 113.45) (size 0.6) (drill 0.3) (layers F.Cu B.Cu) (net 1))
 (segment (start 112.02 102.99) (end 112.02 103.44) (width 0.5) (layer F.Cu) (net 1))
 (segment (start 112.02 103.44) (end 112.02 100.18) (width 0.5) (layer F.Cu) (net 1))
 (segment (start 112.02 100.18) (end 111.58 99.74) (width 0.5) (layer F.Cu) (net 1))
 (segment (start 112.02 104.2164) (end 112.02 103.44) (width 0.5) (layer F.Cu) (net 1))
 (segment (start 112 103.46) (end 112.02 103.44) (width 0.5) (layer F.Cu) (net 1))
 (segment (start 111.58 103) (end 112.02 103.44) (width 0.5) (layer F.Cu) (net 1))
 (segment (start 106.02 118.24) (end 106.02 119.715) (width 0.5) (layer F.Cu) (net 2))
 (segment (start 106.02 119.715) (end 106.555 120.25) (width 0.5) (layer F.Cu) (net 2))
 (segment (start 106.555 120.25) (end 119.5 120.25) (width 0.5) (layer F.Cu) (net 2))
 (segment (start 119.5 120.25) (end 120.02 119.73) (width 0.5) (layer F.Cu) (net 2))
 (segment (start 120.02 119.73) (end 120.02 118.24) (width 0.5) (layer F.Cu) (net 2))
 (segment (start 120.720001 106.590001) (end 120.58 106.45) (width 0.5) (layer F.Cu) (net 2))
 (segment (start 120.58 106.45) (end 118.02 103.89) (width 0.5) (layer F.Cu) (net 2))
 (segment (start 112.72001 106.40499) (end 112.76502 106.45) (width 0.5) (layer F.Cu) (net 2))
 (segment (start 112.76502 106.45) (end 120.58 106.45) (width 0.5) (layer F.Cu) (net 2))
 (segment (start 112.72001 109.285008) (end 112.72001 106.40499) (width 0.5) (layer F.Cu) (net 2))
 (segment (start 120.02 118.24) (end 120.02 116.584998) (width 0.5) (layer F.Cu) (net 2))
 (segment (start 120.02 116.584998) (end 112.72001 109.285008) (width 0.5) (layer F.Cu) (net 2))
 (segment (start 124.96 107.96) (end 123.590001 106.590001) (width 0.5) (layer F.Cu) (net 2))
 (segment (start 123.590001 106.590001) (end 120.720001 106.590001) (width 0.5) (layer F.Cu) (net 2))
 (segment (start 118.02 103.89) (end 118.02 103.44) (width 0.5) (layer F.Cu) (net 2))
 (segment (start 120.02 118.24) (end 120.02 118.69) (width 0.5) (layer F.Cu) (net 2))
 (segment (start 106.02 118.69) (end 106.02 118.24) (width 0.5) (layer F.Cu) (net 2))
 (segment (start 100.665 114.605) (end 98.125 114.605) (width 0.5) (layer F.Cu) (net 2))
 (segment (start 106.02 118.24) (end 104.3 118.24) (width 0.5) (layer F.Cu) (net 2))
 (segment (start 104.3 118.24) (end 100.665 114.605) (width 0.5) (layer F.Cu) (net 2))
 (segment (start 120.02 118.24) (end 120.02 117.79) (width 0.5) (layer F.Cu) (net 2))
 (segment (start 124.77 113.04) (end 124.96 113.04) (width 0.5) (layer F.Cu) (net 2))
 (segment (start 124.96 107.96) (end 124.96 113.04) (width 0.5) (layer F.Cu) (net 2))
 (segment (start 106.02 118.24) (end 106.02 117.79) (width 0.5) (layer F.Cu) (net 2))
 (segment (start 130.04 113.04) (end 130.04 111.102528) (width 0.5) (layer F.Cu) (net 2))
 (segment (start 130.04 111.102528) (end 130.04 107.96) (width 0.5) (layer F.Cu) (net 2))
 (segment (start 124.96 113.04) (end 130.04 113.04) (width 0.5) (layer F.Cu) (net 2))
 (segment (start 116.134 99.36) (end 115.389 98.615) (width 0.5) (layer F.Cu) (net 2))
 (segment (start 110.33 98.615) (end 109.205 99.74) (width 0.5) (layer F.Cu) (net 2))
 (segment (start 109.205 99.74) (end 109.08 99.74) (width 0.5) (layer F.Cu) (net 2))
 (segment (start 115.389 98.615) (end 110.33 98.615) (width 0.5) (layer F.Cu) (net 2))
 (segment (start 116.134 99.36) (end 117.65 99.36) (width 0.5) (layer F.Cu) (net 2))
 (segment (start 117.65 99.36) (end 117.65 103.07) (width 0.5) (layer F.Cu) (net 2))
 (segment (start 117.65 103.07) (end 118.02 103.44) (width 0.5) (layer F.Cu) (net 2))
 (segment (start 114.02 118.24) (end 114.02 117.79) (width 0.5) (layer F.Cu) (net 6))
 (segment (start 114.02 117.79) (end 100.675 104.445) (width 0.5) (layer F.Cu) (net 6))
 (segment (start 100.675 104.445) (end 100.665 104.445) (width 0.5) (layer F.Cu) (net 6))
 (segment (start 114.02 118.24) (end 114.02 117.7) (width 0.5) (layer F.Cu) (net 6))
 (segment (start 110.02 118.24) (end 110.02 116.34) (width 0.5) (layer F.Cu) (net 4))
 (segment (start 110.02 116.34) (end 100.665 106.985) (width 0.5) (layer F.Cu) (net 4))
 (segment (start 110 118.22) (end 110.02 118.24) (width 0.5) (layer F.Cu) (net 4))
 (segment (start 110.02 118.24) (end 110.02 117.79) (width 0.5) (layer F.Cu) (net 4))
 (segment (start 110.02 118.24) (end 110.02 118.69) (width 0.25) (layer F.Cu) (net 4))
 (segment (start 108.02 118.24) (end 108.02 116.765) (width 0.5) (layer F.Cu) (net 3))
 (segment (start 108.02 116.765) (end 100.78 109.525) (width 0.5) (layer F.Cu) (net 3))
 (segment (start 100.78 109.525) (end 100.665 109.525) (width 0.5) (layer F.Cu) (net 3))
 (segment (start 108.02 118.24) (end 108.02 118.550002) (width 0.5) (layer F.Cu) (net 3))
 (segment (start 108.02 118.24) (end 108.02 117.79) (width 0.5) (layer F.Cu) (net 3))
 (segment (start 108.02 118.24) (end 108.02 118.69) (width 0.5) (layer F.Cu) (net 3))
 (segment (start 110.9 116.075) (end 112.02 117.195) (width 0.5) (layer F.Cu) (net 5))
 (segment (start 112.02 117.195) (end 112.02 118.24) (width 0.5) (layer F.Cu) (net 5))
 (segment (start 112.25 114.825) (end 112.15 114.825) (width 0.5) (layer B.Cu) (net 5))
 (segment (start 112.15 114.825) (end 110.9 116.075) (width 0.5) (layer B.Cu) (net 5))
 (via (at 110.9 116.075) (size 0.6) (drill 0.3) (layers F.Cu B.Cu) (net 5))
 (segment (start 110.875 113.225) (end 110.875 113.45) (width 0.5) (layer F.Cu) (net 5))
 (segment (start 110.875 113.45) (end 112.25 114.825) (width 0.5) (layer F.Cu) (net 5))
 (via (at 112.25 114.825) (size 0.6) (drill 0.3) (layers F.Cu B.Cu) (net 5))
 (segment (start 100.665 112.065) (end 109.715 112.065) (width 0.5) (layer B.Cu) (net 5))
 (segment (start 109.715 112.065) (end 110.875 113.225) (width 0.5) (layer B.Cu) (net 5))
 (via (at 110.875 113.225) (size 0.6) (drill 0.3) (layers F.Cu B.Cu) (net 5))
 (segment (start 112.02 118.24) (end 112.02 117.79) (width 0.5) (layer F.Cu) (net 5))
 (segment (start 98.1 99) (end 98.1 104.42) (width 0.5) (layer F.Cu) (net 12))
 (segment (start 98.1 104.42) (end 98.125 104.445) (width 0.5) (layer F.Cu) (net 12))
 (segment (start 105.955 98.925) (end 98.175 98.925) (width 0.5) (layer F.Cu) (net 12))
 (segment (start 98.175 98.925) (end 98.1 99) (width 0.5) (layer F.Cu) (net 12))
 (via (at 98.1 99) (size 0.6) (drill 0.3) (layers F.Cu B.Cu) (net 12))
 (segment (start 110.02 102.99) (end 105.955 98.925) (width 0.5) (layer F.Cu) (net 12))
 (segment (start 110.02 103.44) (end 110.02 102.99) (width 0.5) (layer F.Cu) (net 12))
 (segment (start 110.02 103.44) (end 110.02 103.89) (width 0.25) (layer F.Cu) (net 12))
 (segment (start 110.02 103.89) (end 110 103.91) (width 0.25) (layer F.Cu) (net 12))
 (segment (start 113.075 111.95) (end 104.256399 103.131399) (width 0.5) (layer B.Cu) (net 7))
 (segment (start 104.256399 103.131399) (end 97.494471 103.131399) (width 0.5) (layer B.Cu) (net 7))
 (segment (start 97.261401 106.121401) (end 98.125 106.985) (width 0.5) (layer B.Cu) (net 7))
 (segment (start 97.494471 103.131399) (end 96.811399 103.814471) (width 0.5) (layer B.Cu) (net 7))
 (segment (start 96.811399 103.814471) (end 96.811399 105.671399) (width 0.5) (layer B.Cu) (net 7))
 (segment (start 96.811399 105.671399) (end 97.261401 106.121401) (width 0.5) (layer B.Cu) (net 7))
 (segment (start 116.02 118.24) (end 116.02 114.895) (width 0.5) (layer F.Cu) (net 7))
 (segment (start 116.02 114.895) (end 113.075 111.95) (width 0.5) (layer F.Cu) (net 7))
 (via (at 113.075 111.95) (size 0.6) (drill 0.3) (layers F.Cu B.Cu) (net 7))
 (segment (start 116.02 117.79) (end 116.02 118.24) (width 0.25) (layer F.Cu) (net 7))
 (segment (start 106.55 100.875) (end 108.02 102.345) (width 0.5) (layer F.Cu) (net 13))
 (segment (start 108.02 102.345) (end 108.02 103.44) (width 0.5) (layer F.Cu) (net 13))
 (segment (start 95.725 100.8) (end 106.475 100.8) (width 0.5) (layer B.Cu) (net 13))
 (segment (start 106.475 100.8) (end 106.55 100.875) (width 0.5) (layer B.Cu) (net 13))
 (via (at 106.55 100.875) (size 0.6) (drill 0.3) (layers F.Cu B.Cu) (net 13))
 (segment (start 95.725 108.346314) (end 95.725 107.44087) (width 0.5) (layer F.Cu) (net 13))
 (segment (start 95.725 107.44087) (end 95.725 100.8) (width 0.5) (layer F.Cu) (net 13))
 (via (at 95.725 100.8) (size 0.6) (drill 0.3) (layers F.Cu B.Cu) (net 13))
 (segment (start 98.125 109.525) (end 96.903686 109.525) (width 0.5) (layer F.Cu) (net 13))
 (segment (start 96.903686 109.525) (end 95.725 108.346314) (width 0.5) (layer F.Cu) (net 13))
 (segment (start 107.867831 103.592169) (end 108.02 103.44) (width 0.5) (layer F.Cu) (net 13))
 (segment (start 108.02 103.44) (end 108.02 102.99) (width 0.5) (layer F.Cu) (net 13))
 (segment (start 108.02 103.44) (end 108.02 103.89) (width 0.25) (layer F.Cu) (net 13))
 (segment (start 108.02 103.89) (end 108 103.91) (width 0.25) (layer F.Cu) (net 13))
 (segment (start 105.3 99.875) (end 105.3 102.72) (width 0.5) (layer F.Cu) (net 14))
 (segment (start 105.3 102.72) (end 106.02 103.44) (width 0.5) (layer F.Cu) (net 14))
 (segment (start 96.85 100) (end 105.175 100) (width 0.5) (layer B.Cu) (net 14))
 (via (at 105.3 99.875) (size 0.6) (drill 0.3) (layers F.Cu B.Cu) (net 14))
 (segment (start 105.175 100) (end 105.3 99.875) (width 0.5) (layer B.Cu) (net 14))
 (segment (start 98.125 112.065) (end 94.974999 108.914999) (width 0.5) (layer F.Cu) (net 14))
 (segment (start 94.974999 108.914999) (end 94.974999 100.439999) (width 0.5) (layer F.Cu) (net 14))
 (segment (start 94.974999 100.439999) (end 95.414998 100) (width 0.5) (layer F.Cu) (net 14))
 (segment (start 95.414998 100) (end 96.85 100) (width 0.5) (layer F.Cu) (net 14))
 (via (at 96.85 100) (size 0.6) (drill 0.3) (layers F.Cu B.Cu) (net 14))
 (segment (start 106.02 103.44) (end 106.02 103.89) (width 0.25) (layer F.Cu) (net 14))
 (segment (start 120.02 103.44) (end 123.133602 103.44) (width 0.5) (layer F.Cu) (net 9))
 (segment (start 123.133602 103.44) (end 127.5 107.806398) (width 0.5) (layer F.Cu) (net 9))
 (segment (start 127.5 107.806398) (end 127.5 108.916081) (width 0.5) (layer F.Cu) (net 9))
 (segment (start 127.5 108.916081) (end 127.5 110.5) (width 0.5) (layer F.Cu) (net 9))
 (segment (start 120.19 103.27) (end 120.02 103.44) (width 0.5) (layer F.Cu) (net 9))
 (segment (start 129 100) (end 129 101.175) (width 0.5) (layer B.Cu) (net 8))
 (segment (start 129 101.175) (end 124.725 105.45) (width 0.5) (layer B.Cu) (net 8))
 (segment (start 124.725 105.45) (end 109.325 105.45) (width 0.5) (layer B.Cu) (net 8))
 (segment (start 109.325 105.45) (end 109.25 105.525) (width 0.5) (layer B.Cu) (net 8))
 (segment (start 109.25 105.525) (end 107.85 105.525) (width 0.5) (layer B.Cu) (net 8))
 (segment (start 107.85 105.525) (end 117.975 115.65) (width 0.5) (layer B.Cu) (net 8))
 (segment (start 117.975 115.65) (end 117.975 118.195) (width 0.5) (layer F.Cu) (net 8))
 (segment (start 117.975 118.195) (end 118.02 118.24) (width 0.5) (layer F.Cu) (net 8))
 (via (at 117.975 115.65) (size 0.6) (drill 0.3) (layers F.Cu B.Cu) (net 8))
 (segment (start 118 118.22) (end 118.02 118.24) (width 0.5) (layer F.Cu) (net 8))
 (segment (start 118.02 117.79) (end 118.02 118.24) (width 0.5) (layer F.Cu) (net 8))
 (segment (start 116.3 100.4) (end 122.934998 100.4) (width 0.5) (layer B.Cu) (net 11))
 (segment (start 122.934998 100.4) (end 124.459999 98.874999) (width 0.5) (layer B.Cu) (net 11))
 (segment (start 124.459999 98.874999) (end 125.874999 98.874999) (width 0.5) (layer B.Cu) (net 11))
 (segment (start 125.874999 98.874999) (end 126.325001 99.325001) (width 0.5) (layer B.Cu) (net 11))
 (segment (start 126.325001 99.325001) (end 127 100) (width 0.5) (layer B.Cu) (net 11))
 (segment (start 114.02 103.44) (end 114.02 101.965) (width 0.5) (layer F.Cu) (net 11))
 (segment (start 114.02 101.965) (end 115.585 100.4) (width 0.5) (layer F.Cu) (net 11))
 (segment (start 115.585 100.4) (end 116.3 100.4) (width 0.5) (layer F.Cu) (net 11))
 (via (at 116.3 100.4) (size 0.6) (drill 0.3) (layers F.Cu B.Cu) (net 11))
 (segment (start 114.02 104.376) (end 114.02 103.44) (width 0.5) (layer F.Cu) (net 11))
 (segment (start 116.3 101.4) (end 123.6 101.4) (width 0.5) (layer B.Cu) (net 10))
 (segment (start 123.6 101.4) (end 125 100) (width 0.5) (layer B.Cu) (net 10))
 (segment (start 116.02 103.44) (end 116.02 101.68) (width 0.5) (layer F.Cu) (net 10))
 (segment (start 116.02 101.68) (end 116.3 101.4) (width 0.5) (layer F.Cu) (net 10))
 (via (at 116.3 101.4) (size 0.6) (drill 0.3) (layers F.Cu B.Cu) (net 10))
 (segment (start 116.02 103.89) (end 116.02 103.44) (width 0.5) (layer F.Cu) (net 10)))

